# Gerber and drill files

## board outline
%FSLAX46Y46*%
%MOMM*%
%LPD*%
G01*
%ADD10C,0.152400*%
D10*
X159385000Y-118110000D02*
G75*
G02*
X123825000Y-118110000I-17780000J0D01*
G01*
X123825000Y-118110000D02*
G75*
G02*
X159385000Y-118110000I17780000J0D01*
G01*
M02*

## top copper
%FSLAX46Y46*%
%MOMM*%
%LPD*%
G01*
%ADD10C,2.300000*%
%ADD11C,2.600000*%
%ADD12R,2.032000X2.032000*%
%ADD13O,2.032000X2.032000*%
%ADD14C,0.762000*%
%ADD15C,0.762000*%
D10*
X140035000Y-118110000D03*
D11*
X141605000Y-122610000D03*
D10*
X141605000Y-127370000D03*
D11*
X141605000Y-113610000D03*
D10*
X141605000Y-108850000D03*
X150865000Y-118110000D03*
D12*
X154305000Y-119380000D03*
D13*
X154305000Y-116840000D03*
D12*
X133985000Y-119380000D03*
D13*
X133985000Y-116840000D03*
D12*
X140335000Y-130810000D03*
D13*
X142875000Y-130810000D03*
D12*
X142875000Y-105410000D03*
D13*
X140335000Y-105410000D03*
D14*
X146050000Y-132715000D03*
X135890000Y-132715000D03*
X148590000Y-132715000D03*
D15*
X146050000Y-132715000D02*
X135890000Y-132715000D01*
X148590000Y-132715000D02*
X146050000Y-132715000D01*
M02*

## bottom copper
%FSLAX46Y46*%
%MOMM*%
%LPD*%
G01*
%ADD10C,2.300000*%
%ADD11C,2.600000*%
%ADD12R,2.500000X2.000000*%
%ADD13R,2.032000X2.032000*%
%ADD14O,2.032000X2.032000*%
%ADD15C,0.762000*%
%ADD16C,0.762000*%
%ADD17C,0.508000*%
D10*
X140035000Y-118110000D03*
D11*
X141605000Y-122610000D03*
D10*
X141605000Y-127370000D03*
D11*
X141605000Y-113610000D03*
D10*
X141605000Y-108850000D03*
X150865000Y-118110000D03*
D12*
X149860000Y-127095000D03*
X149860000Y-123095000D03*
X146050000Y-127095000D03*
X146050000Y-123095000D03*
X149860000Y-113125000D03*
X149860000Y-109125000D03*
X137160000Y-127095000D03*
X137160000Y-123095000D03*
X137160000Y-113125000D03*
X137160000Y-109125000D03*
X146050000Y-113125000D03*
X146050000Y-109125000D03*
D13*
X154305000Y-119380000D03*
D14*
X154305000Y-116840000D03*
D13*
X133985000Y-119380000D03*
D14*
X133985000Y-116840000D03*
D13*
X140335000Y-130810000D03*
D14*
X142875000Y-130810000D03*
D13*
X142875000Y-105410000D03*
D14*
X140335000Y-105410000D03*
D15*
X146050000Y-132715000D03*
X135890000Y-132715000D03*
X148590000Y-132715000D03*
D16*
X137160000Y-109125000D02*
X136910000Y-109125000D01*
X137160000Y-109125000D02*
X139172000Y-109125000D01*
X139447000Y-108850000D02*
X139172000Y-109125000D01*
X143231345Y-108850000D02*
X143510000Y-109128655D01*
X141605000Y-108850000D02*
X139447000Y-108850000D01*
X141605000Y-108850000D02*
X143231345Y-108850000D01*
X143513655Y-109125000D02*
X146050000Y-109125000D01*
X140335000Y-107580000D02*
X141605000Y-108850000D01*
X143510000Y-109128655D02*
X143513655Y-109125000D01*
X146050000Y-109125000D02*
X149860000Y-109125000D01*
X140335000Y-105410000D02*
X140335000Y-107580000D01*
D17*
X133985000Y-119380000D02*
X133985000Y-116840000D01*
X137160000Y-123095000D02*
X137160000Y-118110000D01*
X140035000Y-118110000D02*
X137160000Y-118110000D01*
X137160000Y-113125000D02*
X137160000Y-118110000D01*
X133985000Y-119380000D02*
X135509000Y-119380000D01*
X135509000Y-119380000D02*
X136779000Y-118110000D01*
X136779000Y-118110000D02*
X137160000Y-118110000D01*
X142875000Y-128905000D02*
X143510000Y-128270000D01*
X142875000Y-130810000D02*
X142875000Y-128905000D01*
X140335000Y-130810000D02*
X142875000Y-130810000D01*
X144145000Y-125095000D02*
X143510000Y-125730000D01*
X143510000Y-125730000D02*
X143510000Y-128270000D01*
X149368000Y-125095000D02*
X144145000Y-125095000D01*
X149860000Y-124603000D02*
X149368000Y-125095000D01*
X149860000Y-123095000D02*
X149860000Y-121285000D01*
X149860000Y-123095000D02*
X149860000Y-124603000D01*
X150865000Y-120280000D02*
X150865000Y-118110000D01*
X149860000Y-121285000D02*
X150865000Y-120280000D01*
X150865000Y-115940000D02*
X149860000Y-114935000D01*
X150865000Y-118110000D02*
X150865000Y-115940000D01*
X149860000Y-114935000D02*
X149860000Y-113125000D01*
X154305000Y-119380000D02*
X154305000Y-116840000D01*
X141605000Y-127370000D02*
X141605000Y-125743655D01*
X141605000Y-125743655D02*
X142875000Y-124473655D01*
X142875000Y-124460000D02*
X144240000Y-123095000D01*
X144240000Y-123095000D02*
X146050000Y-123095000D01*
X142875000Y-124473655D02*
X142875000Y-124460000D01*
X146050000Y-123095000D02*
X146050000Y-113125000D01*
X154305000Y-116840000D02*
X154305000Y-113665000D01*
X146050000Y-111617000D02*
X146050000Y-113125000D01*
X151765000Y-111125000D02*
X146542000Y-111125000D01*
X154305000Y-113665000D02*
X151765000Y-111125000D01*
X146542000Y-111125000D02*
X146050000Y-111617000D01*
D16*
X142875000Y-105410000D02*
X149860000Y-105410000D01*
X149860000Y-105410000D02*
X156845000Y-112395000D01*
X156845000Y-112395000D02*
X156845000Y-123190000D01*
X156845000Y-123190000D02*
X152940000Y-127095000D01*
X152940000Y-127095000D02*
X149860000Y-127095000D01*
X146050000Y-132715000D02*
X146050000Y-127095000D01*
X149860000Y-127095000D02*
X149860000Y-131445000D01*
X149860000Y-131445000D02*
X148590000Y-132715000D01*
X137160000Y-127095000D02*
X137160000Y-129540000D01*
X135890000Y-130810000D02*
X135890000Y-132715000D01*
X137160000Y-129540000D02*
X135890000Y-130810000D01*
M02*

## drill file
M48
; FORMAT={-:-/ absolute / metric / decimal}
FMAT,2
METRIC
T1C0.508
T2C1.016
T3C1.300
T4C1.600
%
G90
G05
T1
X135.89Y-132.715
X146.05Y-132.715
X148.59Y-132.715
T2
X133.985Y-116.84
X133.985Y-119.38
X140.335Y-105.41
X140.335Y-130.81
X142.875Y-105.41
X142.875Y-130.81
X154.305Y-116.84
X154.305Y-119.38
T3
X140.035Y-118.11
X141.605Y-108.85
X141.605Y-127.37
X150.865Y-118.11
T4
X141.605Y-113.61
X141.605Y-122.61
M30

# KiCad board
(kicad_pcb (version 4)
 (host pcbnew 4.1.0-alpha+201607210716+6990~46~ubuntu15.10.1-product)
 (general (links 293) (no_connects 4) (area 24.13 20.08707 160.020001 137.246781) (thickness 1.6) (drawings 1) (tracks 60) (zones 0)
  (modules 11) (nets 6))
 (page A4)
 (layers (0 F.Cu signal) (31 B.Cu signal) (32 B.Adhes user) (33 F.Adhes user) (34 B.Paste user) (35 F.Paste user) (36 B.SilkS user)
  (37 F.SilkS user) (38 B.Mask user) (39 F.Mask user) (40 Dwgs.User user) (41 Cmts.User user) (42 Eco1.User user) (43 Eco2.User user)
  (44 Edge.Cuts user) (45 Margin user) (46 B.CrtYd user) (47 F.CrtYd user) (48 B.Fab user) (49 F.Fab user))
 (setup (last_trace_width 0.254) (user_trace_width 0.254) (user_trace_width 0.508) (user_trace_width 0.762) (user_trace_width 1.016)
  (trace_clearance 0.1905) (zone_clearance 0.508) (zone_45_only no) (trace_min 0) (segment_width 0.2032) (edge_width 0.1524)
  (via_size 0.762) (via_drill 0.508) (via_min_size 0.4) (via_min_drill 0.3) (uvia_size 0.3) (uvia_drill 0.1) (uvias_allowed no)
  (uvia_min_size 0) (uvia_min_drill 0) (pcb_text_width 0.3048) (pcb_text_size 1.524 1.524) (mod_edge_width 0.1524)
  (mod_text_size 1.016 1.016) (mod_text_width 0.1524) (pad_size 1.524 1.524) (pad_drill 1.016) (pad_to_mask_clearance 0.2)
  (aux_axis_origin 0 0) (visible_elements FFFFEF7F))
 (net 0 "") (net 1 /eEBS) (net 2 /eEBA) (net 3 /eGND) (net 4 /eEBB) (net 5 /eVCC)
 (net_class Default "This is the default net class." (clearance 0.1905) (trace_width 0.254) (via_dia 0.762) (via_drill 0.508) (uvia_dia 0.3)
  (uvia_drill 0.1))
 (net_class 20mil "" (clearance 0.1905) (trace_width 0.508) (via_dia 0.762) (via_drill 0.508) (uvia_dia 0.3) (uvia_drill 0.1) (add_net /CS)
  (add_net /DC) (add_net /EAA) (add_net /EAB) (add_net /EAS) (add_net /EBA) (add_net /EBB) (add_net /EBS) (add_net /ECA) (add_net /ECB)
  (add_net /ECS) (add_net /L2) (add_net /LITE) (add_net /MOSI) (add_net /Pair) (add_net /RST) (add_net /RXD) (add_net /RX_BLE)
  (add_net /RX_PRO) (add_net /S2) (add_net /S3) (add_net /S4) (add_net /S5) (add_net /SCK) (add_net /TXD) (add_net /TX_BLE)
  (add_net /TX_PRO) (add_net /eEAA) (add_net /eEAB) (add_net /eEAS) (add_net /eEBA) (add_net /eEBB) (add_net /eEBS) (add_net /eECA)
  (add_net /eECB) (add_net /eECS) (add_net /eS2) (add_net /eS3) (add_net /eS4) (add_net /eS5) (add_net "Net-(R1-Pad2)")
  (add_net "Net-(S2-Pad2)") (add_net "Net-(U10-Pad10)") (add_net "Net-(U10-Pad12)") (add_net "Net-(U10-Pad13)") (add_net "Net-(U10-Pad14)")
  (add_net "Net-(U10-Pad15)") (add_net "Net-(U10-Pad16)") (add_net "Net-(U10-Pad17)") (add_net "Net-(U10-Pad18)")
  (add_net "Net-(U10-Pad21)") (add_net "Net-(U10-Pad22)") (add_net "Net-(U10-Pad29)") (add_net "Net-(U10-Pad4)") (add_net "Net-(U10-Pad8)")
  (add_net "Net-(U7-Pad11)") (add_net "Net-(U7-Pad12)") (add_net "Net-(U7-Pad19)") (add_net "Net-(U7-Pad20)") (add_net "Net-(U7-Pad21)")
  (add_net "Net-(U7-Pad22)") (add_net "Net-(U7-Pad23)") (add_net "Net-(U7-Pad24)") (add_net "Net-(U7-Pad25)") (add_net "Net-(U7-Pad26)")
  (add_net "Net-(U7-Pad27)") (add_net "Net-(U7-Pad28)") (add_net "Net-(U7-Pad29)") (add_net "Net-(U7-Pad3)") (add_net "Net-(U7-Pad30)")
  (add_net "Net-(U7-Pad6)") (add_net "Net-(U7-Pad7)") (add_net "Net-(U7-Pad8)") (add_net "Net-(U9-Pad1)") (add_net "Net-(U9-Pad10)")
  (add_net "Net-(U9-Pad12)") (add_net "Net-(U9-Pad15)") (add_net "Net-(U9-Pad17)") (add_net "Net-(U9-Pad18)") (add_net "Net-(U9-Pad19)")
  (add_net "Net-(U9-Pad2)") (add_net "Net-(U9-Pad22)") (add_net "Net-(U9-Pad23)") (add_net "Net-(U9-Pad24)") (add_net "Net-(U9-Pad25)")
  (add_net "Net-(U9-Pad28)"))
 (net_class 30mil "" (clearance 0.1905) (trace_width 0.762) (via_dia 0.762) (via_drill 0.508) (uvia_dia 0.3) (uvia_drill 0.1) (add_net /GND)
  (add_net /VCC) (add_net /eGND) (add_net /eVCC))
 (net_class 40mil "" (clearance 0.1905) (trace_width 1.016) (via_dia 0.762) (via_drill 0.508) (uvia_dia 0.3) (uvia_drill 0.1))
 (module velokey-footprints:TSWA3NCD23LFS (layer F.Cu) (at 141.605 118.11 90)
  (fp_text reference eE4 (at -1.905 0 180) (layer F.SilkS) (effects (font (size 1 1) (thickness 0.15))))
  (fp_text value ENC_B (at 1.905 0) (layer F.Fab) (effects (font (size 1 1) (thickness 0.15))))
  (pad 4 thru_hole circle (at 0 -1.57 90) (size 2.3 2.3) (drill 1.3) (layers *.Cu *.Mask F.SilkS) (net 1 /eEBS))
  (pad 5 thru_hole circle (at -4.5 0 90) (size 2.6 2.6) (drill 1.6) (layers *.Cu *.Mask F.SilkS))
  (pad 1 thru_hole circle (at -9.26 0 90) (size 2.3 2.3) (drill 1.3) (layers *.Cu *.Mask F.SilkS) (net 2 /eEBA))
  (pad 6 thru_hole circle (at 4.5 0 90) (size 2.6 2.6) (drill 1.6) (layers *.Cu *.Mask F.SilkS))
  (pad 2 thru_hole circle (at 9.26 0 90) (size 2.3 2.3) (drill 1.3) (layers *.Cu *.Mask F.SilkS) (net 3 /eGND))
  (pad 3 thru_hole circle (at 0 9.26 90) (size 2.3 2.3) (drill 1.3) (layers *.Cu *.Mask F.SilkS) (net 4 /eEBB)))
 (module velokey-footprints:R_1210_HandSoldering (layer B.Cu) (at 149.86 125.095 90)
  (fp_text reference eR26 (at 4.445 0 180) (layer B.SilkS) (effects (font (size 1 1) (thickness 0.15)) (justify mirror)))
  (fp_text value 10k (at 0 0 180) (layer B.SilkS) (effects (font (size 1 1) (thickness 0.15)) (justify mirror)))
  (pad 1 smd rect (at -2 0 90) (size 2 2.5) (layers B.Cu B.Paste B.Mask) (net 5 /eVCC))
  (pad 2 smd rect (at 2 0 90) (size 2 2.5) (layers B.Cu B.Paste B.Mask) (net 4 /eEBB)))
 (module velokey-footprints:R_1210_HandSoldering (layer B.Cu) (at 146.05 125.095 90)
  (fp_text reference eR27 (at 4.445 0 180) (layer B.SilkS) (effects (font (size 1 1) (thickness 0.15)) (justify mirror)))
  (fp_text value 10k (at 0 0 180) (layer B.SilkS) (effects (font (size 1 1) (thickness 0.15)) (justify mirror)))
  (pad 1 smd rect (at -2 0 90) (size 2 2.5) (layers B.Cu B.Paste B.Mask) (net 5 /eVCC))
  (pad 2 smd rect (at 2 0 90) (size 2 2.5) (layers B.Cu B.Paste B.Mask) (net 2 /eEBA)))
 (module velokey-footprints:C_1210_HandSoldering (layer B.Cu) (at 149.86 111.125 90)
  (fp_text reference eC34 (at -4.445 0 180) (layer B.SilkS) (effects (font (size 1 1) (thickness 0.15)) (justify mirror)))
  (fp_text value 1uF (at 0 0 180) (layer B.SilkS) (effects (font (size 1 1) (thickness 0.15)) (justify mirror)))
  (pad 1 smd rect (at -2 0 90) (size 2 2.5) (layers B.Cu B.Paste B.Mask) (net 4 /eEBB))
  (pad 2 smd rect (at 2 0 90) (size 2 2.5) (layers B.Cu B.Paste B.Mask) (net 3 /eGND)))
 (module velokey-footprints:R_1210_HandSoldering (layer B.Cu) (at 137.16 125.095 90)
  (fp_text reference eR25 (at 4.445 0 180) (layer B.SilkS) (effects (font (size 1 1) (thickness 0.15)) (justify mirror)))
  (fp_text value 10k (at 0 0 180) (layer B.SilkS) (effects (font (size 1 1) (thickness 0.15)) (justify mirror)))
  (pad 1 smd rect (at -2 0 90) (size 2 2.5) (layers B.Cu B.Paste B.Mask) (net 5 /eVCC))
  (pad 2 smd rect (at 2 0 90) (size 2 2.5) (layers B.Cu B.Paste B.Mask) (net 1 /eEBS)))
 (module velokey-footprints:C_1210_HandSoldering (layer B.Cu) (at 137.16 111.125 90)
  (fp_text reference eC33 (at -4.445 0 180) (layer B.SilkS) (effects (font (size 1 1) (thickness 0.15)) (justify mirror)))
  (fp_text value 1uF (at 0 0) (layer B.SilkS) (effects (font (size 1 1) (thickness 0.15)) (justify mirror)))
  (pad 1 smd rect (at -2 0 90) (size 2 2.5) (layers B.Cu B.Paste B.Mask) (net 1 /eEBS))
  (pad 2 smd rect (at 2 0 90) (size 2 2.5) (layers B.Cu B.Paste B.Mask) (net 3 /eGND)))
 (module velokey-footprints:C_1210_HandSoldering (layer B.Cu) (at 146.05 111.125 90)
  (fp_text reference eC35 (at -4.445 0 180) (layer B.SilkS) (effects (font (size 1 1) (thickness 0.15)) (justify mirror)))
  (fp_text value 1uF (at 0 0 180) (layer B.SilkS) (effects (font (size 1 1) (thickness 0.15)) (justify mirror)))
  (pad 1 smd rect (at -2 0 90) (size 2 2.5) (layers B.Cu B.Paste B.Mask) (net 2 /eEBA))
  (pad 2 smd rect (at 2 0 90) (size 2 2.5) (layers B.Cu B.Paste B.Mask) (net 3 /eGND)))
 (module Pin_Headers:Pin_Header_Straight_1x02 (layer F.Cu) (at 154.305 119.38 180)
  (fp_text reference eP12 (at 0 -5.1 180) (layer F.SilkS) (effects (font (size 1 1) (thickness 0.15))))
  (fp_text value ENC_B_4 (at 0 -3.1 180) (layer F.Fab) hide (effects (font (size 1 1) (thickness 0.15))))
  (pad 1 thru_hole rect (at 0 0 180) (size 2.032 2.032) (drill 1.016) (layers *.Cu *.Mask F.SilkS) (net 2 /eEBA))
  (pad 2 thru_hole oval (at 0 2.54 180) (size 2.032 2.032) (drill 1.016) (layers *.Cu *.Mask F.SilkS) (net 2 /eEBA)))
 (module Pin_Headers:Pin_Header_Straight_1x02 (layer F.Cu) (at 133.985 119.38 180)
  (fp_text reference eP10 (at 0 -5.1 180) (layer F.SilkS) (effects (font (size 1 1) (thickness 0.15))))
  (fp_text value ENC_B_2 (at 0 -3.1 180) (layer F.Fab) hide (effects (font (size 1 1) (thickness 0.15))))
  (pad 1 thru_hole rect (at 0 0 180) (size 2.032 2.032) (drill 1.016) (layers *.Cu *.Mask F.SilkS) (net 1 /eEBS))
  (pad 2 thru_hole oval (at 0 2.54 180) (size 2.032 2.032) (drill 1.016) (layers *.Cu *.Mask F.SilkS) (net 1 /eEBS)))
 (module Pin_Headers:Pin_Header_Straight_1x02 (layer F.Cu) (at 140.335 130.81 90)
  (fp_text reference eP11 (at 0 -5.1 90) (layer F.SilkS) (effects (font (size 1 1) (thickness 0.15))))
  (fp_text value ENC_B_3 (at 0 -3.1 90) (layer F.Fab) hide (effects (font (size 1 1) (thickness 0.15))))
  (pad 1 thru_hole rect (at 0 0 90) (size 2.032 2.032) (drill 1.016) (layers *.Cu *.Mask F.SilkS) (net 4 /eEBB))
  (pad 2 thru_hole oval (at 0 2.54 90) (size 2.032 2.032) (drill 1.016) (layers *.Cu *.Mask F.SilkS) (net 4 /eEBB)))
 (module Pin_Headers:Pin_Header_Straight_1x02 (layer F.Cu) (at 142.875 105.41 270)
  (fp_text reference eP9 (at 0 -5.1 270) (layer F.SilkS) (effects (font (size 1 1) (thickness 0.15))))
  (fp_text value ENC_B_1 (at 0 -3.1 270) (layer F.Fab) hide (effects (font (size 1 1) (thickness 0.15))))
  (pad 1 thru_hole rect (at 0 0 270) (size 2.032 2.032) (drill 1.016) (layers *.Cu *.Mask F.SilkS) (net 5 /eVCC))
  (pad 2 thru_hole oval (at 0 2.54 270) (size 2.032 2.032) (drill 1.016) (layers *.Cu *.Mask F.SilkS) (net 3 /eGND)))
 (gr_circle (center 141.605 118.11) (end 123.825 118.11) (layer Edge.Cuts) (width 0.1524))
 (segment (start 137.16 109.125) (end 136.91 109.125) (width 0.762) (layer B.Cu) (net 3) (status 30))
 (segment (start 137.16 109.125) (end 139.172 109.125) (width 0.762) (layer B.Cu) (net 3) (status 10))
 (segment (start 139.447 108.85) (end 139.172 109.125) (width 0.762) (layer B.Cu) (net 3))
 (segment (start 143.231345 108.85) (end 143.51 109.128655) (width 0.762) (layer B.Cu) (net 3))
 (segment (start 141.605 108.85) (end 139.447 108.85) (width 0.762) (layer B.Cu) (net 3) (status 10))
 (segment (start 141.605 108.85) (end 143.231345 108.85) (width 0.762) (layer B.Cu) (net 3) (status 10))
 (segment (start 143.513655 109.125) (end 146.05 109.125) (width 0.762) (layer B.Cu) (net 3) (status 20))
 (segment (start 140.335 107.58) (end 141.605 108.85) (width 0.762) (layer B.Cu) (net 3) (status 20))
 (segment (start 143.51 109.128655) (end 143.513655 109.125) (width 0.762) (layer B.Cu) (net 3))
 (segment (start 146.05 109.125) (end 149.86 109.125) (width 0.762) (layer B.Cu) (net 3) (status 30))
 (segment (start 140.335 105.41) (end 140.335 107.58) (width 0.762) (layer B.Cu) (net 3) (status 10))
 (segment (start 133.985 119.38) (end 133.985 116.84) (width 0.508) (layer B.Cu) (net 1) (status 30))
 (segment (start 137.16 123.095) (end 137.16 118.11) (width 0.508) (layer B.Cu) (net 1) (status 10))
 (segment (start 140.035 118.11) (end 137.16 118.11) (width 0.508) (layer B.Cu) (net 1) (status 10))
 (segment (start 137.16 113.125) (end 137.16 118.11) (width 0.508) (layer B.Cu) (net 1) (status 10))
 (segment (start 133.985 119.38) (end 135.509 119.38) (width 0.508) (layer B.Cu) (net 1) (status 10))
 (segment (start 135.509 119.38) (end 136.779 118.11) (width 0.508) (layer B.Cu) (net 1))
 (segment (start 136.779 118.11) (end 137.16 118.11) (width 0.508) (layer B.Cu) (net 1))
 (segment (start 142.875 128.905) (end 143.51 128.27) (width 0.508) (layer B.Cu) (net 4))
 (segment (start 142.875 130.81) (end 142.875 128.905) (width 0.508) (layer B.Cu) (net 4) (status 10))
 (segment (start 140.335 130.81) (end 142.875 130.81) (width 0.508) (layer B.Cu) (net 4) (status 30))
 (segment (start 144.145 125.095) (end 143.51 125.73) (width 0.508) (layer B.Cu) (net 4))
 (segment (start 143.51 125.73) (end 143.51 128.27) (width 0.508) (layer B.Cu) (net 4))
 (segment (start 149.368 125.095) (end 144.145 125.095) (width 0.508) (layer B.Cu) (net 4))
 (segment (start 149.86 124.603) (end 149.368 125.095) (width 0.508) (layer B.Cu) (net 4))
 (segment (start 149.86 123.095) (end 149.86 121.285) (width 0.508) (layer B.Cu) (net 4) (status 10))
 (segment (start 149.86 123.095) (end 149.86 124.603) (width 0.508) (layer B.Cu) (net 4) (status 10))
 (segment (start 150.865 120.28) (end 150.865 118.11) (width 0.508) (layer B.Cu) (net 4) (status 20))
 (segment (start 149.86 121.285) (end 150.865 120.28) (width 0.508) (layer B.Cu) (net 4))
 (segment (start 150.865 115.94) (end 149.86 114.935) (width 0.508) (layer B.Cu) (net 4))
 (segment (start 150.865 118.11) (end 150.865 115.94) (width 0.508) (layer B.Cu) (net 4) (status 10))
 (segment (start 149.86 114.935) (end 149.86 113.125) (width 0.508) (layer B.Cu) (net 4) (status 20))
 (segment (start 154.305 119.38) (end 154.305 116.84) (width 0.508) (layer B.Cu) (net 2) (status 30))
 (segment (start 141.605 127.37) (end 141.605 125.743655) (width 0.508) (layer B.Cu) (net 2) (status 10))
 (segment (start 141.605 125.743655) (end 142.875 124.473655) (width 0.508) (layer B.Cu) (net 2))
 (segment (start 142.875 124.46) (end 144.24 123.095) (width 0.508) (layer B.Cu) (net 2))
 (segment (start 144.24 123.095) (end 146.05 123.095) (width 0.508) (layer B.Cu) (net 2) (status 20))
 (segment (start 142.875 124.473655) (end 142.875 124.46) (width 0.508) (layer B.Cu) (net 2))
 (segment (start 146.05 123.095) (end 146.05 113.125) (width 0.508) (layer B.Cu) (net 2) (status 30))
 (segment (start 154.305 116.84) (end 154.305 113.665) (width 0.508) (layer B.Cu) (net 2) (status 10))
 (segment (start 146.05 111.617) (end 146.05 113.125) (width 0.508) (layer B.Cu) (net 2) (status 20))
 (segment (start 151.765 111.125) (end 146.542 111.125) (width 0.508) (layer B.Cu) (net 2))
 (segment (start 154.305 113.665) (end 151.765 111.125) (width 0.508) (layer B.Cu) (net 2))
 (segment (start 146.542 111.125) (end 146.05 111.617) (width 0.508) (layer B.Cu) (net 2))
 (segment (start 142.875 105.41) (end 149.86 105.41) (width 0.762) (layer B.Cu) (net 5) (status 10))
 (segment (start 149.86 105.41) (end 156.845 112.395) (width 0.762) (layer B.Cu) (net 5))
 (segment (start 156.845 112.395) (end 156.845 123.19) (width 0.762) (layer B.Cu) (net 5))
 (segment (start 156.845 123.19) (end 152.94 127.095) (width 0.762) (layer B.Cu) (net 5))
 (segment (start 152.94 127.095) (end 149.86 127.095) (width 0.762) (layer B.Cu) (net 5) (status 20))
 (segment (start 146.05 132.715) (end 146.05 127.095) (width 0.762) (layer B.Cu) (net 5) (status 20))
 (segment (start 149.86 127.095) (end 149.86 131.445) (width 0.762) (layer B.Cu) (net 5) (status 10))
 (segment (start 149.86 131.445) (end 148.59 132.715) (width 0.762) (layer B.Cu) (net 5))
 (segment (start 137.16 127.095) (end 137.16 129.54) (width 0.762) (layer B.Cu) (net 5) (status 10))
 (segment (start 135.89 130.81) (end 135.89 132.715) (width 0.762) (layer B.Cu) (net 5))
 (segment (start 137.16 129.54) (end 135.89 130.81) (width 0.762) (layer B.Cu) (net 5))
 (segment (start 146.05 132.715) (end 135.89 132.715) (width 0.762) (layer F.Cu) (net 5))
 (segment (start 148.59 132.715) (end 146.05 132.715) (width 0.762) (layer F.Cu) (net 5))
 (via (at 146.05 132.715) (size 0.762) (drill 0.508) (layers F.Cu B.Cu) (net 5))
 (via (at 135.89 132.715) (size 0.762) (drill 0.508) (layers F.Cu B.Cu) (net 5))
 (via (at 148.59 132.715) (size 0.762) (drill 0.508) (layers F.Cu B.Cu) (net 5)))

